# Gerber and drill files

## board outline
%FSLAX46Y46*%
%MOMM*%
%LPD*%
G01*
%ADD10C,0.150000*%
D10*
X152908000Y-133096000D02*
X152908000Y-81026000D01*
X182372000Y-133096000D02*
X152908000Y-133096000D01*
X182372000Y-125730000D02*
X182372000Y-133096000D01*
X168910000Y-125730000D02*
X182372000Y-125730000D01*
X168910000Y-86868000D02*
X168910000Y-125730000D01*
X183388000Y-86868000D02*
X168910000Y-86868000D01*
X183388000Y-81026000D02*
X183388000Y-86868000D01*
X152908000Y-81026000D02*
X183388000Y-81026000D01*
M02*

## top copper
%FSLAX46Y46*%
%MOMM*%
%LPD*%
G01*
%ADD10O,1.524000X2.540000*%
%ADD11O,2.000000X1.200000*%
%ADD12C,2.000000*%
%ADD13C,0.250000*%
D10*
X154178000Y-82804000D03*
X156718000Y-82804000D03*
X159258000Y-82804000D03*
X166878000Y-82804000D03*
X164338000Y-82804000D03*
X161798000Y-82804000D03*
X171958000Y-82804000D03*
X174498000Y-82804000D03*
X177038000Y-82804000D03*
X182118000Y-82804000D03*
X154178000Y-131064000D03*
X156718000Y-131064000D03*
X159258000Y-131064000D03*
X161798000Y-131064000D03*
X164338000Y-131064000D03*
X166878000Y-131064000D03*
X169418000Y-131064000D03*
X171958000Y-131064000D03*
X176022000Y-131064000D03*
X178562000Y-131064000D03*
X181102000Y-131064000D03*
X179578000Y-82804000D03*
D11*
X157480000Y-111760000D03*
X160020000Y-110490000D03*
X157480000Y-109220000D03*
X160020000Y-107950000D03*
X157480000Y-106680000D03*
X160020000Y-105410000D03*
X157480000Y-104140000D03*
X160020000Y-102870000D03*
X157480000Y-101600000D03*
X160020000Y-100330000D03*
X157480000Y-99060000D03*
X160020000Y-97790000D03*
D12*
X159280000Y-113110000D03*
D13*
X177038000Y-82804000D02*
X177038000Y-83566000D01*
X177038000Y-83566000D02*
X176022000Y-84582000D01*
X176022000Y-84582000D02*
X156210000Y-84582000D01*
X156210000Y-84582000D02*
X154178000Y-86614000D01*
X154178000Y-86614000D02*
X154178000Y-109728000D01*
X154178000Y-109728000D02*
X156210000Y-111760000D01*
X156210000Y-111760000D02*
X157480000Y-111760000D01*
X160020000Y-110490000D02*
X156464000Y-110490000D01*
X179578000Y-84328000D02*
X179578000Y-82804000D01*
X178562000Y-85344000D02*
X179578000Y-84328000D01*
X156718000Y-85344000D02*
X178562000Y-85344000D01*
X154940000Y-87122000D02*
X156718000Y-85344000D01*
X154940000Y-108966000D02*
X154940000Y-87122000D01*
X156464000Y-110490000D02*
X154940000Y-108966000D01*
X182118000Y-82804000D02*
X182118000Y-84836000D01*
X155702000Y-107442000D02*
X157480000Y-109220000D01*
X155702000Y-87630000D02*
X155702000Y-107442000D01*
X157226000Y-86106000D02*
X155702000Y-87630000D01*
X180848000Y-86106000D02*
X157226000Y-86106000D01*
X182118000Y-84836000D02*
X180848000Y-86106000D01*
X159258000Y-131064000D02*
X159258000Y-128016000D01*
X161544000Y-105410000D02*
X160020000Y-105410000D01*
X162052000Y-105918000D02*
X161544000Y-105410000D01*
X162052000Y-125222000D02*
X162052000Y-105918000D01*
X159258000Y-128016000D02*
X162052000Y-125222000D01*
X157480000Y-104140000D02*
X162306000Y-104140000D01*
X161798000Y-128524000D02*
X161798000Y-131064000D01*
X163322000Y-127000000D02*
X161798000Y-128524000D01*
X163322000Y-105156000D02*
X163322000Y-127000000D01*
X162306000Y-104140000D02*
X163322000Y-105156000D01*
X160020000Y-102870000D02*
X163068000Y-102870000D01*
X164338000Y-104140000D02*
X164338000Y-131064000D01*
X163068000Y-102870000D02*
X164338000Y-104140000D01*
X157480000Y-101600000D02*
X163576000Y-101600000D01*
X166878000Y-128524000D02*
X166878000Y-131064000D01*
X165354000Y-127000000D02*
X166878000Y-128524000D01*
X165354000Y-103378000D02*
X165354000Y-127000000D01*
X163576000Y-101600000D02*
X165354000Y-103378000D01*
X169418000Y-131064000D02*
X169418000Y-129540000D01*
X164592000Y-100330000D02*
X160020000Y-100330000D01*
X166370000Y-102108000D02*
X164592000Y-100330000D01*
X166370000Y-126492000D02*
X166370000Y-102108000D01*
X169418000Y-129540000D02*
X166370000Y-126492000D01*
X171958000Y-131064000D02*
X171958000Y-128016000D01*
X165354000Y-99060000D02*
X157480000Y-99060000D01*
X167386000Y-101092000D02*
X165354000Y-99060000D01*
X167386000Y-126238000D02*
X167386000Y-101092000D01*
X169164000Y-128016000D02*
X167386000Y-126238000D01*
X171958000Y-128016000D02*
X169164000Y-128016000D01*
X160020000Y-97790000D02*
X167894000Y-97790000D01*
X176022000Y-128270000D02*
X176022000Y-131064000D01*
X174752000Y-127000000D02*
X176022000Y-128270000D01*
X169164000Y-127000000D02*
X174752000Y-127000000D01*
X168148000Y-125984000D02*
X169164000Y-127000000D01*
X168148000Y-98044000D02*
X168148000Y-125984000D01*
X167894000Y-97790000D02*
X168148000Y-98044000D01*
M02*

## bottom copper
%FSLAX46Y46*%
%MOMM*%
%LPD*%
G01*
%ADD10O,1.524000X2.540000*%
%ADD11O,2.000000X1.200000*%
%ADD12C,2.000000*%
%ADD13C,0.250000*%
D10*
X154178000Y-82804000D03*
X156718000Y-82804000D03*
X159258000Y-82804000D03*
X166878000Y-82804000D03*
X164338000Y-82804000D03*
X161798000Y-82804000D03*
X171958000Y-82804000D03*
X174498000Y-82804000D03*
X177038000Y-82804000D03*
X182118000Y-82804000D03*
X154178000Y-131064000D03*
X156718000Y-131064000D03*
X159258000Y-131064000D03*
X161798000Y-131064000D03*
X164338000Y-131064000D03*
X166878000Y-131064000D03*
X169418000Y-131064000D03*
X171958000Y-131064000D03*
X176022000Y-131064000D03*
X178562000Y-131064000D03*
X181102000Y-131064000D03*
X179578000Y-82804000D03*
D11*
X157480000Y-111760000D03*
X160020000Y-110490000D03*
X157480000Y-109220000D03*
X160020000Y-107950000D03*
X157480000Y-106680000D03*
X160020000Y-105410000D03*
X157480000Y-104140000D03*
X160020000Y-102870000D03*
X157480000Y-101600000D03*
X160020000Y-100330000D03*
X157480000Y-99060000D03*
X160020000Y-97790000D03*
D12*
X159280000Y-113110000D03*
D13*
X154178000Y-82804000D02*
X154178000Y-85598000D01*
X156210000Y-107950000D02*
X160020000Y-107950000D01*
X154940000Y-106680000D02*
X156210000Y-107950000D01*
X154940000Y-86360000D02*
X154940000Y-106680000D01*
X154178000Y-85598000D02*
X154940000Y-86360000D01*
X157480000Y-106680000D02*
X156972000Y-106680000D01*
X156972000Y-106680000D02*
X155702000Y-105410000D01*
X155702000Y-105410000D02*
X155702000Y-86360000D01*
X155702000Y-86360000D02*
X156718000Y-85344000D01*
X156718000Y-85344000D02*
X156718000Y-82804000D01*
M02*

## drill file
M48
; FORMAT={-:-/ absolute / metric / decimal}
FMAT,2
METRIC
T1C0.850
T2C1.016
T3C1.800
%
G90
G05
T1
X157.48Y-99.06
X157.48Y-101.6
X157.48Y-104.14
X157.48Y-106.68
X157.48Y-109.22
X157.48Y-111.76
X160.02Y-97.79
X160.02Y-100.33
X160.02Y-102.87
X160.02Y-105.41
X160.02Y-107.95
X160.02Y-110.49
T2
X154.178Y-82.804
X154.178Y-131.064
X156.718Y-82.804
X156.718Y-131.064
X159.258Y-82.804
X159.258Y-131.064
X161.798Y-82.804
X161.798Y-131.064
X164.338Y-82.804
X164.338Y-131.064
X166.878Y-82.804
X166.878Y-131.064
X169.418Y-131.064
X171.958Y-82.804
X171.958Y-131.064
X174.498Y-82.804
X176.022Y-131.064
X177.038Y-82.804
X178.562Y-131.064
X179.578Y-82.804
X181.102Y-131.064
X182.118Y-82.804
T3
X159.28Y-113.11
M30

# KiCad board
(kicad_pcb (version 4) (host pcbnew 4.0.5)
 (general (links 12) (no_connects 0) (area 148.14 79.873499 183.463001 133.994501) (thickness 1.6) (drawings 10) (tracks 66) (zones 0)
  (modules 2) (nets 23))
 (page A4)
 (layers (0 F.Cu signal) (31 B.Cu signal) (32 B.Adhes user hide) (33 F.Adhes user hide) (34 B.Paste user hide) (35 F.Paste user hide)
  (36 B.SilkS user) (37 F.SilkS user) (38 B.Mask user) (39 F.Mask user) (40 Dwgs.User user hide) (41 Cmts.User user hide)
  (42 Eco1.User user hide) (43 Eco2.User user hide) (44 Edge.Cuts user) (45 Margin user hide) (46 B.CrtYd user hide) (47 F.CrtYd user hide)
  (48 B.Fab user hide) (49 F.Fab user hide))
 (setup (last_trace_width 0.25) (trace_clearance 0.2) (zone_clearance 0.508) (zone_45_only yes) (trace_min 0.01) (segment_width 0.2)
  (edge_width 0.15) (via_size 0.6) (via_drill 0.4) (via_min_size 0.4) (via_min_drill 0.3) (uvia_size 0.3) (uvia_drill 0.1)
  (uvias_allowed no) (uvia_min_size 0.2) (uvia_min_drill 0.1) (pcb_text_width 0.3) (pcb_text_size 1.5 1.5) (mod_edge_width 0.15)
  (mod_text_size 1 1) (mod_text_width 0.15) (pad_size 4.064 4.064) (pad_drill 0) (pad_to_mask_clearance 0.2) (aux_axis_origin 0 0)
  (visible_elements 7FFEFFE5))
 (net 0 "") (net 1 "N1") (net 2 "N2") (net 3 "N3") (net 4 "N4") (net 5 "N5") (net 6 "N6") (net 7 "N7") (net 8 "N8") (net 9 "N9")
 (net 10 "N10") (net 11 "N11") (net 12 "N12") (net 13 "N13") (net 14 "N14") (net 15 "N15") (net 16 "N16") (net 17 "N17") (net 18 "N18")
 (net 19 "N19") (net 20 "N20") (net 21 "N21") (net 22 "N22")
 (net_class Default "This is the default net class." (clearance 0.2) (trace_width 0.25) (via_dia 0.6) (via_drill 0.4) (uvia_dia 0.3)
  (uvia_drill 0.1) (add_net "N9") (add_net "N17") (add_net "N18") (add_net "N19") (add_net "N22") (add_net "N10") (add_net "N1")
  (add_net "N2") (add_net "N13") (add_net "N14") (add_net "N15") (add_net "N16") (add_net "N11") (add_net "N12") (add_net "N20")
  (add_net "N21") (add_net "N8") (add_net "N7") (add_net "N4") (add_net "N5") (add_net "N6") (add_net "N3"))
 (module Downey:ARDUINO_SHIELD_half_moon (layer F.Cu) (at 148.59 104.14 270)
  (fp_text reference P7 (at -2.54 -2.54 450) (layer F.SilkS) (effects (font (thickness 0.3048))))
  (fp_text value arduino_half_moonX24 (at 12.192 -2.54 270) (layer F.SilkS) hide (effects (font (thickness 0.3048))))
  (pad 11 thru_hole oval (at -21.336 -5.588 270) (size 2.54 1.524) (drill 1.016) (layers *.Cu *.Mask F.SilkS) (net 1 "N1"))
  (pad 10 thru_hole oval (at -21.336 -8.128 270) (size 2.54 1.524) (drill 1.016) (layers *.Cu *.Mask F.SilkS) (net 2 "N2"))
  (pad 9 thru_hole oval (at -21.336 -10.668 270) (size 2.54 1.524) (drill 1.016) (layers *.Cu *.Mask F.SilkS) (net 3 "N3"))
  (pad 6 thru_hole oval (at -21.336 -18.288 270) (size 2.54 1.524) (drill 1.016) (layers *.Cu *.Mask F.SilkS) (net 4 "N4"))
  (pad 7 thru_hole oval (at -21.336 -15.748 270) (size 2.54 1.524) (drill 1.016) (layers *.Cu *.Mask F.SilkS) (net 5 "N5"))
  (pad 8 thru_hole oval (at -21.336 -13.208 270) (size 2.54 1.524) (drill 1.016) (layers *.Cu *.Mask F.SilkS) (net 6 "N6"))
  (pad 5 thru_hole oval (at -21.336 -23.368 270) (size 2.54 1.524) (drill 1.016) (layers *.Cu *.Mask F.SilkS) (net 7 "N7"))
  (pad 4 thru_hole oval (at -21.336 -25.908 270) (size 2.54 1.524) (drill 1.016) (layers *.Cu *.Mask F.SilkS) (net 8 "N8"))
  (pad 3 thru_hole oval (at -21.336 -28.448 270) (size 2.54 1.524) (drill 1.016) (layers *.Cu *.Mask F.SilkS) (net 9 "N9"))
  (pad 1 thru_hole oval (at -21.336 -33.528 270) (size 2.54 1.524) (drill 1.016) (layers *.Cu *.Mask F.SilkS) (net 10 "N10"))
  (pad 12 thru_hole oval (at 26.924 -5.588 270) (size 2.54 1.524) (drill 1.016) (layers *.Cu *.Mask F.SilkS) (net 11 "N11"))
  (pad 13 thru_hole oval (at 26.924 -8.128 270) (size 2.54 1.524) (drill 1.016) (layers *.Cu *.Mask F.SilkS) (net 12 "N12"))
  (pad 14 thru_hole oval (at 26.924 -10.668 270) (size 2.54 1.524) (drill 1.016) (layers *.Cu *.Mask F.SilkS) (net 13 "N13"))
  (pad 15 thru_hole oval (at 26.924 -13.208 270) (size 2.54 1.524) (drill 1.016) (layers *.Cu *.Mask F.SilkS) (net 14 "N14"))
  (pad 16 thru_hole oval (at 26.924 -15.748 270) (size 2.54 1.524) (drill 1.016) (layers *.Cu *.Mask F.SilkS) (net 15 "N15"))
  (pad 17 thru_hole oval (at 26.924 -18.288 270) (size 2.54 1.524) (drill 1.016) (layers *.Cu *.Mask F.SilkS) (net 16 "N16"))
  (pad 18 thru_hole oval (at 26.924 -20.828 270) (size 2.54 1.524) (drill 1.016) (layers *.Cu *.Mask F.SilkS) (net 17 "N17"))
  (pad 19 thru_hole oval (at 26.924 -23.368 270) (size 2.54 1.524) (drill 1.016) (layers *.Cu *.Mask F.SilkS) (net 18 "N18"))
  (pad 20 thru_hole oval (at 26.924 -27.432 270) (size 2.54 1.524) (drill 1.016) (layers *.Cu *.Mask F.SilkS) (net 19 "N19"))
  (pad 21 thru_hole oval (at 26.924 -29.972 270) (size 2.54 1.524) (drill 1.016) (layers *.Cu *.Mask F.SilkS) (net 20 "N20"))
  (pad 22 thru_hole oval (at 26.924 -32.512 270) (size 2.54 1.524) (drill 1.016) (layers *.Cu *.Mask F.SilkS) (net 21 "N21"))
  (pad 2 thru_hole oval (at -21.336 -30.988 270) (size 2.54 1.524) (drill 1.016) (layers *.Cu *.Mask F.SilkS) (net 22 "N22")))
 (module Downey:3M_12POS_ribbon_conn (layer F.Cu) (at 158.75 105.41 90)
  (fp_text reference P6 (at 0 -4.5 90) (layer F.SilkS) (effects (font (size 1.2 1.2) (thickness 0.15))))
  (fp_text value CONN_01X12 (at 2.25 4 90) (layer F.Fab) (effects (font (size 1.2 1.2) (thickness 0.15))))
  (pad 1 thru_hole oval (at -6.35 -1.27 90) (size 1.2 2) (drill 0.85) (layers *.Cu *.Mask) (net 9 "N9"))
  (pad 2 thru_hole oval (at -5.08 1.27 90) (size 1.2 2) (drill 0.85) (layers *.Cu *.Mask) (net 22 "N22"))
  (pad 3 thru_hole oval (at -3.81 -1.27 90) (size 1.2 2) (drill 0.85) (layers *.Cu *.Mask) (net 10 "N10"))
  (pad 4 thru_hole oval (at -2.54 1.27 90) (size 1.2 2) (drill 0.85) (layers *.Cu *.Mask) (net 1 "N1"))
  (pad 5 thru_hole oval (at -1.27 -1.27 90) (size 1.2 2) (drill 0.85) (layers *.Cu *.Mask) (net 2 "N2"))
  (pad 6 thru_hole oval (at 0 1.27 90) (size 1.2 2) (drill 0.85) (layers *.Cu *.Mask) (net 13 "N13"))
  (pad 7 thru_hole oval (at 1.27 -1.27 90) (size 1.2 2) (drill 0.85) (layers *.Cu *.Mask) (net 14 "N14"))
  (pad 8 thru_hole oval (at 2.54 1.27 90) (size 1.2 2) (drill 0.85) (layers *.Cu *.Mask) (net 15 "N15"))
  (pad 9 thru_hole oval (at 3.81 -1.27 90) (size 1.2 2) (drill 0.85) (layers *.Cu *.Mask) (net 16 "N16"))
  (pad 10 thru_hole oval (at 5.08 1.27 90) (size 1.2 2) (drill 0.85) (layers *.Cu *.Mask) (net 17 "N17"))
  (pad 11 thru_hole oval (at 6.35 -1.27 90) (size 1.2 2) (drill 0.85) (layers *.Cu *.Mask) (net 18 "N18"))
  (pad 12 thru_hole oval (at 7.62 1.27 90) (size 1.2 2) (drill 0.85) (layers *.Cu *.Mask) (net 19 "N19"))
  (pad "" np_thru_hole circle (at -7.7 0.53 90) (size 2 2) (drill 1.8) (layers *.Cu *.Mask)))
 (gr_line (start 152.908 133.096) (end 152.908 81.026) (angle 90) (layer Edge.Cuts) (width 0.15))
 (gr_line (start 182.372 133.096) (end 152.908 133.096) (angle 90) (layer Edge.Cuts) (width 0.15))
 (gr_line (start 182.372 125.73) (end 182.372 133.096) (angle 90) (layer Edge.Cuts) (width 0.15))
 (gr_line (start 168.91 125.73) (end 182.372 125.73) (angle 90) (layer Edge.Cuts) (width 0.15))
 (gr_line (start 168.91 86.868) (end 168.91 125.73) (angle 90) (layer Edge.Cuts) (width 0.15))
 (gr_line (start 183.388 86.868) (end 168.91 86.868) (angle 90) (layer Edge.Cuts) (width 0.15))
 (gr_line (start 183.388 81.026) (end 183.388 86.868) (angle 90) (layer Edge.Cuts) (width 0.15))
 (gr_line (start 152.908 81.026) (end 183.388 81.026) (angle 90) (layer Edge.Cuts) (width 0.15))
 (segment (start 177.038 82.804) (end 177.038 83.566) (width 0.25) (layer F.Cu) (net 9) (status C00000))
 (segment (start 177.038 83.566) (end 176.022 84.582) (width 0.25) (layer F.Cu) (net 9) (status 400000))
 (segment (start 176.022 84.582) (end 156.21 84.582) (width 0.25) (layer F.Cu) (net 9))
 (segment (start 156.21 84.582) (end 154.178 86.614) (width 0.25) (layer F.Cu) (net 9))
 (segment (start 154.178 86.614) (end 154.178 109.728) (width 0.25) (layer F.Cu) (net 9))
 (segment (start 154.178 109.728) (end 156.21 111.76) (width 0.25) (layer F.Cu) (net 9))
 (segment (start 156.21 111.76) (end 157.48 111.76) (width 0.25) (layer F.Cu) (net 9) (status 800000))
 (segment (start 160.02 110.49) (end 156.464 110.49) (width 0.25) (layer F.Cu) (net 22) (status 400000))
 (segment (start 179.578 84.328) (end 179.578 82.804) (width 0.25) (layer F.Cu) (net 22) (status 800000))
 (segment (start 178.562 85.344) (end 179.578 84.328) (width 0.25) (layer F.Cu) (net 22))
 (segment (start 156.718 85.344) (end 178.562 85.344) (width 0.25) (layer F.Cu) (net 22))
 (segment (start 154.94 87.122) (end 156.718 85.344) (width 0.25) (layer F.Cu) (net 22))
 (segment (start 154.94 108.966) (end 154.94 87.122) (width 0.25) (layer F.Cu) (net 22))
 (segment (start 156.464 110.49) (end 154.94 108.966) (width 0.25) (layer F.Cu) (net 22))
 (segment (start 182.118 82.804) (end 182.118 84.836) (width 0.25) (layer F.Cu) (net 10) (status 400000))
 (segment (start 155.702 107.442) (end 157.48 109.22) (width 0.25) (layer F.Cu) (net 10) (status 800000))
 (segment (start 155.702 87.63) (end 155.702 107.442) (width 0.25) (layer F.Cu) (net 10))
 (segment (start 157.226 86.106) (end 155.702 87.63) (width 0.25) (layer F.Cu) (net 10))
 (segment (start 180.848 86.106) (end 157.226 86.106) (width 0.25) (layer F.Cu) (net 10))
 (segment (start 182.118 84.836) (end 180.848 86.106) (width 0.25) (layer F.Cu) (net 10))
 (segment (start 154.178 82.804) (end 154.178 85.598) (width 0.25) (layer B.Cu) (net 1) (status 400000))
 (segment (start 156.21 107.95) (end 160.02 107.95) (width 0.25) (layer B.Cu) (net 1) (status 800000))
 (segment (start 154.94 106.68) (end 156.21 107.95) (width 0.25) (layer B.Cu) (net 1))
 (segment (start 154.94 86.36) (end 154.94 106.68) (width 0.25) (layer B.Cu) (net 1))
 (segment (start 154.178 85.598) (end 154.94 86.36) (width 0.25) (layer B.Cu) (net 1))
 (segment (start 157.48 106.68) (end 156.972 106.68) (width 0.25) (layer B.Cu) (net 2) (status C00000))
 (segment (start 156.972 106.68) (end 155.702 105.41) (width 0.25) (layer B.Cu) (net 2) (status 400000))
 (segment (start 155.702 105.41) (end 155.702 86.36) (width 0.25) (layer B.Cu) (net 2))
 (segment (start 155.702 86.36) (end 156.718 85.344) (width 0.25) (layer B.Cu) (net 2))
 (segment (start 156.718 85.344) (end 156.718 82.804) (width 0.25) (layer B.Cu) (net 2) (status 800000))
 (segment (start 159.258 131.064) (end 159.258 128.016) (width 0.25) (layer F.Cu) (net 13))
 (segment (start 161.544 105.41) (end 160.02 105.41) (width 0.25) (layer F.Cu) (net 13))
 (segment (start 162.052 105.918) (end 161.544 105.41) (width 0.25) (layer F.Cu) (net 13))
 (segment (start 162.052 125.222) (end 162.052 105.918) (width 0.25) (layer F.Cu) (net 13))
 (segment (start 159.258 128.016) (end 162.052 125.222) (width 0.25) (layer F.Cu) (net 13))
 (segment (start 157.48 104.14) (end 162.306 104.14) (width 0.25) (layer F.Cu) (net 14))
 (segment (start 161.798 128.524) (end 161.798 131.064) (width 0.25) (layer F.Cu) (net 14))
 (segment (start 163.322 127) (end 161.798 128.524) (width 0.25) (layer F.Cu) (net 14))
 (segment (start 163.322 105.156) (end 163.322 127) (width 0.25) (layer F.Cu) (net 14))
 (segment (start 162.306 104.14) (end 163.322 105.156) (width 0.25) (layer F.Cu) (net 14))
 (segment (start 160.02 102.87) (end 163.068 102.87) (width 0.25) (layer F.Cu) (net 15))
 (segment (start 164.338 104.14) (end 164.338 131.064) (width 0.25) (layer F.Cu) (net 15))
 (segment (start 163.068 102.87) (end 164.338 104.14) (width 0.25) (layer F.Cu) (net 15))
 (segment (start 157.48 101.6) (end 163.576 101.6) (width 0.25) (layer F.Cu) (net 16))
 (segment (start 166.878 128.524) (end 166.878 131.064) (width 0.25) (layer F.Cu) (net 16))
 (segment (start 165.354 127) (end 166.878 128.524) (width 0.25) (layer F.Cu) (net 16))
 (segment (start 165.354 103.378) (end 165.354 127) (width 0.25) (layer F.Cu) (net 16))
 (segment (start 163.576 101.6) (end 165.354 103.378) (width 0.25) (layer F.Cu) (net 16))
 (segment (start 169.418 131.064) (end 169.418 129.54) (width 0.25) (layer F.Cu) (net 17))
 (segment (start 164.592 100.33) (end 160.02 100.33) (width 0.25) (layer F.Cu) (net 17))
 (segment (start 166.37 102.108) (end 164.592 100.33) (width 0.25) (layer F.Cu) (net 17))
 (segment (start 166.37 126.492) (end 166.37 102.108) (width 0.25) (layer F.Cu) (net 17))
 (segment (start 169.418 129.54) (end 166.37 126.492) (width 0.25) (layer F.Cu) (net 17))
 (segment (start 171.958 131.064) (end 171.958 128.016) (width 0.25) (layer F.Cu) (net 18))
 (segment (start 165.354 99.06) (end 157.48 99.06) (width 0.25) (layer F.Cu) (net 18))
 (segment (start 167.386 101.092) (end 165.354 99.06) (width 0.25) (layer F.Cu) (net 18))
 (segment (start 167.386 126.238) (end 167.386 101.092) (width 0.25) (layer F.Cu) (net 18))
 (segment (start 169.164 128.016) (end 167.386 126.238) (width 0.25) (layer F.Cu) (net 18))
 (segment (start 171.958 128.016) (end 169.164 128.016) (width 0.25) (layer F.Cu) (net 18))
 (segment (start 160.02 97.79) (end 167.894 97.79) (width 0.25) (layer F.Cu) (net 19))
 (segment (start 176.022 128.27) (end 176.022 131.064) (width 0.25) (layer F.Cu) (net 19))
 (segment (start 174.752 127) (end 176.022 128.27) (width 0.25) (layer F.Cu) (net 19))
 (segment (start 169.164 127) (end 174.752 127) (width 0.25) (layer F.Cu) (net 19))
 (segment (start 168.148 125.984) (end 169.164 127) (width 0.25) (layer F.Cu) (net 19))
 (segment (start 168.148 98.044) (end 168.148 125.984) (width 0.25) (layer F.Cu) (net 19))
 (segment (start 167.894 97.79) (end 168.148 98.044) (width 0.25) (layer F.Cu) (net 19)))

